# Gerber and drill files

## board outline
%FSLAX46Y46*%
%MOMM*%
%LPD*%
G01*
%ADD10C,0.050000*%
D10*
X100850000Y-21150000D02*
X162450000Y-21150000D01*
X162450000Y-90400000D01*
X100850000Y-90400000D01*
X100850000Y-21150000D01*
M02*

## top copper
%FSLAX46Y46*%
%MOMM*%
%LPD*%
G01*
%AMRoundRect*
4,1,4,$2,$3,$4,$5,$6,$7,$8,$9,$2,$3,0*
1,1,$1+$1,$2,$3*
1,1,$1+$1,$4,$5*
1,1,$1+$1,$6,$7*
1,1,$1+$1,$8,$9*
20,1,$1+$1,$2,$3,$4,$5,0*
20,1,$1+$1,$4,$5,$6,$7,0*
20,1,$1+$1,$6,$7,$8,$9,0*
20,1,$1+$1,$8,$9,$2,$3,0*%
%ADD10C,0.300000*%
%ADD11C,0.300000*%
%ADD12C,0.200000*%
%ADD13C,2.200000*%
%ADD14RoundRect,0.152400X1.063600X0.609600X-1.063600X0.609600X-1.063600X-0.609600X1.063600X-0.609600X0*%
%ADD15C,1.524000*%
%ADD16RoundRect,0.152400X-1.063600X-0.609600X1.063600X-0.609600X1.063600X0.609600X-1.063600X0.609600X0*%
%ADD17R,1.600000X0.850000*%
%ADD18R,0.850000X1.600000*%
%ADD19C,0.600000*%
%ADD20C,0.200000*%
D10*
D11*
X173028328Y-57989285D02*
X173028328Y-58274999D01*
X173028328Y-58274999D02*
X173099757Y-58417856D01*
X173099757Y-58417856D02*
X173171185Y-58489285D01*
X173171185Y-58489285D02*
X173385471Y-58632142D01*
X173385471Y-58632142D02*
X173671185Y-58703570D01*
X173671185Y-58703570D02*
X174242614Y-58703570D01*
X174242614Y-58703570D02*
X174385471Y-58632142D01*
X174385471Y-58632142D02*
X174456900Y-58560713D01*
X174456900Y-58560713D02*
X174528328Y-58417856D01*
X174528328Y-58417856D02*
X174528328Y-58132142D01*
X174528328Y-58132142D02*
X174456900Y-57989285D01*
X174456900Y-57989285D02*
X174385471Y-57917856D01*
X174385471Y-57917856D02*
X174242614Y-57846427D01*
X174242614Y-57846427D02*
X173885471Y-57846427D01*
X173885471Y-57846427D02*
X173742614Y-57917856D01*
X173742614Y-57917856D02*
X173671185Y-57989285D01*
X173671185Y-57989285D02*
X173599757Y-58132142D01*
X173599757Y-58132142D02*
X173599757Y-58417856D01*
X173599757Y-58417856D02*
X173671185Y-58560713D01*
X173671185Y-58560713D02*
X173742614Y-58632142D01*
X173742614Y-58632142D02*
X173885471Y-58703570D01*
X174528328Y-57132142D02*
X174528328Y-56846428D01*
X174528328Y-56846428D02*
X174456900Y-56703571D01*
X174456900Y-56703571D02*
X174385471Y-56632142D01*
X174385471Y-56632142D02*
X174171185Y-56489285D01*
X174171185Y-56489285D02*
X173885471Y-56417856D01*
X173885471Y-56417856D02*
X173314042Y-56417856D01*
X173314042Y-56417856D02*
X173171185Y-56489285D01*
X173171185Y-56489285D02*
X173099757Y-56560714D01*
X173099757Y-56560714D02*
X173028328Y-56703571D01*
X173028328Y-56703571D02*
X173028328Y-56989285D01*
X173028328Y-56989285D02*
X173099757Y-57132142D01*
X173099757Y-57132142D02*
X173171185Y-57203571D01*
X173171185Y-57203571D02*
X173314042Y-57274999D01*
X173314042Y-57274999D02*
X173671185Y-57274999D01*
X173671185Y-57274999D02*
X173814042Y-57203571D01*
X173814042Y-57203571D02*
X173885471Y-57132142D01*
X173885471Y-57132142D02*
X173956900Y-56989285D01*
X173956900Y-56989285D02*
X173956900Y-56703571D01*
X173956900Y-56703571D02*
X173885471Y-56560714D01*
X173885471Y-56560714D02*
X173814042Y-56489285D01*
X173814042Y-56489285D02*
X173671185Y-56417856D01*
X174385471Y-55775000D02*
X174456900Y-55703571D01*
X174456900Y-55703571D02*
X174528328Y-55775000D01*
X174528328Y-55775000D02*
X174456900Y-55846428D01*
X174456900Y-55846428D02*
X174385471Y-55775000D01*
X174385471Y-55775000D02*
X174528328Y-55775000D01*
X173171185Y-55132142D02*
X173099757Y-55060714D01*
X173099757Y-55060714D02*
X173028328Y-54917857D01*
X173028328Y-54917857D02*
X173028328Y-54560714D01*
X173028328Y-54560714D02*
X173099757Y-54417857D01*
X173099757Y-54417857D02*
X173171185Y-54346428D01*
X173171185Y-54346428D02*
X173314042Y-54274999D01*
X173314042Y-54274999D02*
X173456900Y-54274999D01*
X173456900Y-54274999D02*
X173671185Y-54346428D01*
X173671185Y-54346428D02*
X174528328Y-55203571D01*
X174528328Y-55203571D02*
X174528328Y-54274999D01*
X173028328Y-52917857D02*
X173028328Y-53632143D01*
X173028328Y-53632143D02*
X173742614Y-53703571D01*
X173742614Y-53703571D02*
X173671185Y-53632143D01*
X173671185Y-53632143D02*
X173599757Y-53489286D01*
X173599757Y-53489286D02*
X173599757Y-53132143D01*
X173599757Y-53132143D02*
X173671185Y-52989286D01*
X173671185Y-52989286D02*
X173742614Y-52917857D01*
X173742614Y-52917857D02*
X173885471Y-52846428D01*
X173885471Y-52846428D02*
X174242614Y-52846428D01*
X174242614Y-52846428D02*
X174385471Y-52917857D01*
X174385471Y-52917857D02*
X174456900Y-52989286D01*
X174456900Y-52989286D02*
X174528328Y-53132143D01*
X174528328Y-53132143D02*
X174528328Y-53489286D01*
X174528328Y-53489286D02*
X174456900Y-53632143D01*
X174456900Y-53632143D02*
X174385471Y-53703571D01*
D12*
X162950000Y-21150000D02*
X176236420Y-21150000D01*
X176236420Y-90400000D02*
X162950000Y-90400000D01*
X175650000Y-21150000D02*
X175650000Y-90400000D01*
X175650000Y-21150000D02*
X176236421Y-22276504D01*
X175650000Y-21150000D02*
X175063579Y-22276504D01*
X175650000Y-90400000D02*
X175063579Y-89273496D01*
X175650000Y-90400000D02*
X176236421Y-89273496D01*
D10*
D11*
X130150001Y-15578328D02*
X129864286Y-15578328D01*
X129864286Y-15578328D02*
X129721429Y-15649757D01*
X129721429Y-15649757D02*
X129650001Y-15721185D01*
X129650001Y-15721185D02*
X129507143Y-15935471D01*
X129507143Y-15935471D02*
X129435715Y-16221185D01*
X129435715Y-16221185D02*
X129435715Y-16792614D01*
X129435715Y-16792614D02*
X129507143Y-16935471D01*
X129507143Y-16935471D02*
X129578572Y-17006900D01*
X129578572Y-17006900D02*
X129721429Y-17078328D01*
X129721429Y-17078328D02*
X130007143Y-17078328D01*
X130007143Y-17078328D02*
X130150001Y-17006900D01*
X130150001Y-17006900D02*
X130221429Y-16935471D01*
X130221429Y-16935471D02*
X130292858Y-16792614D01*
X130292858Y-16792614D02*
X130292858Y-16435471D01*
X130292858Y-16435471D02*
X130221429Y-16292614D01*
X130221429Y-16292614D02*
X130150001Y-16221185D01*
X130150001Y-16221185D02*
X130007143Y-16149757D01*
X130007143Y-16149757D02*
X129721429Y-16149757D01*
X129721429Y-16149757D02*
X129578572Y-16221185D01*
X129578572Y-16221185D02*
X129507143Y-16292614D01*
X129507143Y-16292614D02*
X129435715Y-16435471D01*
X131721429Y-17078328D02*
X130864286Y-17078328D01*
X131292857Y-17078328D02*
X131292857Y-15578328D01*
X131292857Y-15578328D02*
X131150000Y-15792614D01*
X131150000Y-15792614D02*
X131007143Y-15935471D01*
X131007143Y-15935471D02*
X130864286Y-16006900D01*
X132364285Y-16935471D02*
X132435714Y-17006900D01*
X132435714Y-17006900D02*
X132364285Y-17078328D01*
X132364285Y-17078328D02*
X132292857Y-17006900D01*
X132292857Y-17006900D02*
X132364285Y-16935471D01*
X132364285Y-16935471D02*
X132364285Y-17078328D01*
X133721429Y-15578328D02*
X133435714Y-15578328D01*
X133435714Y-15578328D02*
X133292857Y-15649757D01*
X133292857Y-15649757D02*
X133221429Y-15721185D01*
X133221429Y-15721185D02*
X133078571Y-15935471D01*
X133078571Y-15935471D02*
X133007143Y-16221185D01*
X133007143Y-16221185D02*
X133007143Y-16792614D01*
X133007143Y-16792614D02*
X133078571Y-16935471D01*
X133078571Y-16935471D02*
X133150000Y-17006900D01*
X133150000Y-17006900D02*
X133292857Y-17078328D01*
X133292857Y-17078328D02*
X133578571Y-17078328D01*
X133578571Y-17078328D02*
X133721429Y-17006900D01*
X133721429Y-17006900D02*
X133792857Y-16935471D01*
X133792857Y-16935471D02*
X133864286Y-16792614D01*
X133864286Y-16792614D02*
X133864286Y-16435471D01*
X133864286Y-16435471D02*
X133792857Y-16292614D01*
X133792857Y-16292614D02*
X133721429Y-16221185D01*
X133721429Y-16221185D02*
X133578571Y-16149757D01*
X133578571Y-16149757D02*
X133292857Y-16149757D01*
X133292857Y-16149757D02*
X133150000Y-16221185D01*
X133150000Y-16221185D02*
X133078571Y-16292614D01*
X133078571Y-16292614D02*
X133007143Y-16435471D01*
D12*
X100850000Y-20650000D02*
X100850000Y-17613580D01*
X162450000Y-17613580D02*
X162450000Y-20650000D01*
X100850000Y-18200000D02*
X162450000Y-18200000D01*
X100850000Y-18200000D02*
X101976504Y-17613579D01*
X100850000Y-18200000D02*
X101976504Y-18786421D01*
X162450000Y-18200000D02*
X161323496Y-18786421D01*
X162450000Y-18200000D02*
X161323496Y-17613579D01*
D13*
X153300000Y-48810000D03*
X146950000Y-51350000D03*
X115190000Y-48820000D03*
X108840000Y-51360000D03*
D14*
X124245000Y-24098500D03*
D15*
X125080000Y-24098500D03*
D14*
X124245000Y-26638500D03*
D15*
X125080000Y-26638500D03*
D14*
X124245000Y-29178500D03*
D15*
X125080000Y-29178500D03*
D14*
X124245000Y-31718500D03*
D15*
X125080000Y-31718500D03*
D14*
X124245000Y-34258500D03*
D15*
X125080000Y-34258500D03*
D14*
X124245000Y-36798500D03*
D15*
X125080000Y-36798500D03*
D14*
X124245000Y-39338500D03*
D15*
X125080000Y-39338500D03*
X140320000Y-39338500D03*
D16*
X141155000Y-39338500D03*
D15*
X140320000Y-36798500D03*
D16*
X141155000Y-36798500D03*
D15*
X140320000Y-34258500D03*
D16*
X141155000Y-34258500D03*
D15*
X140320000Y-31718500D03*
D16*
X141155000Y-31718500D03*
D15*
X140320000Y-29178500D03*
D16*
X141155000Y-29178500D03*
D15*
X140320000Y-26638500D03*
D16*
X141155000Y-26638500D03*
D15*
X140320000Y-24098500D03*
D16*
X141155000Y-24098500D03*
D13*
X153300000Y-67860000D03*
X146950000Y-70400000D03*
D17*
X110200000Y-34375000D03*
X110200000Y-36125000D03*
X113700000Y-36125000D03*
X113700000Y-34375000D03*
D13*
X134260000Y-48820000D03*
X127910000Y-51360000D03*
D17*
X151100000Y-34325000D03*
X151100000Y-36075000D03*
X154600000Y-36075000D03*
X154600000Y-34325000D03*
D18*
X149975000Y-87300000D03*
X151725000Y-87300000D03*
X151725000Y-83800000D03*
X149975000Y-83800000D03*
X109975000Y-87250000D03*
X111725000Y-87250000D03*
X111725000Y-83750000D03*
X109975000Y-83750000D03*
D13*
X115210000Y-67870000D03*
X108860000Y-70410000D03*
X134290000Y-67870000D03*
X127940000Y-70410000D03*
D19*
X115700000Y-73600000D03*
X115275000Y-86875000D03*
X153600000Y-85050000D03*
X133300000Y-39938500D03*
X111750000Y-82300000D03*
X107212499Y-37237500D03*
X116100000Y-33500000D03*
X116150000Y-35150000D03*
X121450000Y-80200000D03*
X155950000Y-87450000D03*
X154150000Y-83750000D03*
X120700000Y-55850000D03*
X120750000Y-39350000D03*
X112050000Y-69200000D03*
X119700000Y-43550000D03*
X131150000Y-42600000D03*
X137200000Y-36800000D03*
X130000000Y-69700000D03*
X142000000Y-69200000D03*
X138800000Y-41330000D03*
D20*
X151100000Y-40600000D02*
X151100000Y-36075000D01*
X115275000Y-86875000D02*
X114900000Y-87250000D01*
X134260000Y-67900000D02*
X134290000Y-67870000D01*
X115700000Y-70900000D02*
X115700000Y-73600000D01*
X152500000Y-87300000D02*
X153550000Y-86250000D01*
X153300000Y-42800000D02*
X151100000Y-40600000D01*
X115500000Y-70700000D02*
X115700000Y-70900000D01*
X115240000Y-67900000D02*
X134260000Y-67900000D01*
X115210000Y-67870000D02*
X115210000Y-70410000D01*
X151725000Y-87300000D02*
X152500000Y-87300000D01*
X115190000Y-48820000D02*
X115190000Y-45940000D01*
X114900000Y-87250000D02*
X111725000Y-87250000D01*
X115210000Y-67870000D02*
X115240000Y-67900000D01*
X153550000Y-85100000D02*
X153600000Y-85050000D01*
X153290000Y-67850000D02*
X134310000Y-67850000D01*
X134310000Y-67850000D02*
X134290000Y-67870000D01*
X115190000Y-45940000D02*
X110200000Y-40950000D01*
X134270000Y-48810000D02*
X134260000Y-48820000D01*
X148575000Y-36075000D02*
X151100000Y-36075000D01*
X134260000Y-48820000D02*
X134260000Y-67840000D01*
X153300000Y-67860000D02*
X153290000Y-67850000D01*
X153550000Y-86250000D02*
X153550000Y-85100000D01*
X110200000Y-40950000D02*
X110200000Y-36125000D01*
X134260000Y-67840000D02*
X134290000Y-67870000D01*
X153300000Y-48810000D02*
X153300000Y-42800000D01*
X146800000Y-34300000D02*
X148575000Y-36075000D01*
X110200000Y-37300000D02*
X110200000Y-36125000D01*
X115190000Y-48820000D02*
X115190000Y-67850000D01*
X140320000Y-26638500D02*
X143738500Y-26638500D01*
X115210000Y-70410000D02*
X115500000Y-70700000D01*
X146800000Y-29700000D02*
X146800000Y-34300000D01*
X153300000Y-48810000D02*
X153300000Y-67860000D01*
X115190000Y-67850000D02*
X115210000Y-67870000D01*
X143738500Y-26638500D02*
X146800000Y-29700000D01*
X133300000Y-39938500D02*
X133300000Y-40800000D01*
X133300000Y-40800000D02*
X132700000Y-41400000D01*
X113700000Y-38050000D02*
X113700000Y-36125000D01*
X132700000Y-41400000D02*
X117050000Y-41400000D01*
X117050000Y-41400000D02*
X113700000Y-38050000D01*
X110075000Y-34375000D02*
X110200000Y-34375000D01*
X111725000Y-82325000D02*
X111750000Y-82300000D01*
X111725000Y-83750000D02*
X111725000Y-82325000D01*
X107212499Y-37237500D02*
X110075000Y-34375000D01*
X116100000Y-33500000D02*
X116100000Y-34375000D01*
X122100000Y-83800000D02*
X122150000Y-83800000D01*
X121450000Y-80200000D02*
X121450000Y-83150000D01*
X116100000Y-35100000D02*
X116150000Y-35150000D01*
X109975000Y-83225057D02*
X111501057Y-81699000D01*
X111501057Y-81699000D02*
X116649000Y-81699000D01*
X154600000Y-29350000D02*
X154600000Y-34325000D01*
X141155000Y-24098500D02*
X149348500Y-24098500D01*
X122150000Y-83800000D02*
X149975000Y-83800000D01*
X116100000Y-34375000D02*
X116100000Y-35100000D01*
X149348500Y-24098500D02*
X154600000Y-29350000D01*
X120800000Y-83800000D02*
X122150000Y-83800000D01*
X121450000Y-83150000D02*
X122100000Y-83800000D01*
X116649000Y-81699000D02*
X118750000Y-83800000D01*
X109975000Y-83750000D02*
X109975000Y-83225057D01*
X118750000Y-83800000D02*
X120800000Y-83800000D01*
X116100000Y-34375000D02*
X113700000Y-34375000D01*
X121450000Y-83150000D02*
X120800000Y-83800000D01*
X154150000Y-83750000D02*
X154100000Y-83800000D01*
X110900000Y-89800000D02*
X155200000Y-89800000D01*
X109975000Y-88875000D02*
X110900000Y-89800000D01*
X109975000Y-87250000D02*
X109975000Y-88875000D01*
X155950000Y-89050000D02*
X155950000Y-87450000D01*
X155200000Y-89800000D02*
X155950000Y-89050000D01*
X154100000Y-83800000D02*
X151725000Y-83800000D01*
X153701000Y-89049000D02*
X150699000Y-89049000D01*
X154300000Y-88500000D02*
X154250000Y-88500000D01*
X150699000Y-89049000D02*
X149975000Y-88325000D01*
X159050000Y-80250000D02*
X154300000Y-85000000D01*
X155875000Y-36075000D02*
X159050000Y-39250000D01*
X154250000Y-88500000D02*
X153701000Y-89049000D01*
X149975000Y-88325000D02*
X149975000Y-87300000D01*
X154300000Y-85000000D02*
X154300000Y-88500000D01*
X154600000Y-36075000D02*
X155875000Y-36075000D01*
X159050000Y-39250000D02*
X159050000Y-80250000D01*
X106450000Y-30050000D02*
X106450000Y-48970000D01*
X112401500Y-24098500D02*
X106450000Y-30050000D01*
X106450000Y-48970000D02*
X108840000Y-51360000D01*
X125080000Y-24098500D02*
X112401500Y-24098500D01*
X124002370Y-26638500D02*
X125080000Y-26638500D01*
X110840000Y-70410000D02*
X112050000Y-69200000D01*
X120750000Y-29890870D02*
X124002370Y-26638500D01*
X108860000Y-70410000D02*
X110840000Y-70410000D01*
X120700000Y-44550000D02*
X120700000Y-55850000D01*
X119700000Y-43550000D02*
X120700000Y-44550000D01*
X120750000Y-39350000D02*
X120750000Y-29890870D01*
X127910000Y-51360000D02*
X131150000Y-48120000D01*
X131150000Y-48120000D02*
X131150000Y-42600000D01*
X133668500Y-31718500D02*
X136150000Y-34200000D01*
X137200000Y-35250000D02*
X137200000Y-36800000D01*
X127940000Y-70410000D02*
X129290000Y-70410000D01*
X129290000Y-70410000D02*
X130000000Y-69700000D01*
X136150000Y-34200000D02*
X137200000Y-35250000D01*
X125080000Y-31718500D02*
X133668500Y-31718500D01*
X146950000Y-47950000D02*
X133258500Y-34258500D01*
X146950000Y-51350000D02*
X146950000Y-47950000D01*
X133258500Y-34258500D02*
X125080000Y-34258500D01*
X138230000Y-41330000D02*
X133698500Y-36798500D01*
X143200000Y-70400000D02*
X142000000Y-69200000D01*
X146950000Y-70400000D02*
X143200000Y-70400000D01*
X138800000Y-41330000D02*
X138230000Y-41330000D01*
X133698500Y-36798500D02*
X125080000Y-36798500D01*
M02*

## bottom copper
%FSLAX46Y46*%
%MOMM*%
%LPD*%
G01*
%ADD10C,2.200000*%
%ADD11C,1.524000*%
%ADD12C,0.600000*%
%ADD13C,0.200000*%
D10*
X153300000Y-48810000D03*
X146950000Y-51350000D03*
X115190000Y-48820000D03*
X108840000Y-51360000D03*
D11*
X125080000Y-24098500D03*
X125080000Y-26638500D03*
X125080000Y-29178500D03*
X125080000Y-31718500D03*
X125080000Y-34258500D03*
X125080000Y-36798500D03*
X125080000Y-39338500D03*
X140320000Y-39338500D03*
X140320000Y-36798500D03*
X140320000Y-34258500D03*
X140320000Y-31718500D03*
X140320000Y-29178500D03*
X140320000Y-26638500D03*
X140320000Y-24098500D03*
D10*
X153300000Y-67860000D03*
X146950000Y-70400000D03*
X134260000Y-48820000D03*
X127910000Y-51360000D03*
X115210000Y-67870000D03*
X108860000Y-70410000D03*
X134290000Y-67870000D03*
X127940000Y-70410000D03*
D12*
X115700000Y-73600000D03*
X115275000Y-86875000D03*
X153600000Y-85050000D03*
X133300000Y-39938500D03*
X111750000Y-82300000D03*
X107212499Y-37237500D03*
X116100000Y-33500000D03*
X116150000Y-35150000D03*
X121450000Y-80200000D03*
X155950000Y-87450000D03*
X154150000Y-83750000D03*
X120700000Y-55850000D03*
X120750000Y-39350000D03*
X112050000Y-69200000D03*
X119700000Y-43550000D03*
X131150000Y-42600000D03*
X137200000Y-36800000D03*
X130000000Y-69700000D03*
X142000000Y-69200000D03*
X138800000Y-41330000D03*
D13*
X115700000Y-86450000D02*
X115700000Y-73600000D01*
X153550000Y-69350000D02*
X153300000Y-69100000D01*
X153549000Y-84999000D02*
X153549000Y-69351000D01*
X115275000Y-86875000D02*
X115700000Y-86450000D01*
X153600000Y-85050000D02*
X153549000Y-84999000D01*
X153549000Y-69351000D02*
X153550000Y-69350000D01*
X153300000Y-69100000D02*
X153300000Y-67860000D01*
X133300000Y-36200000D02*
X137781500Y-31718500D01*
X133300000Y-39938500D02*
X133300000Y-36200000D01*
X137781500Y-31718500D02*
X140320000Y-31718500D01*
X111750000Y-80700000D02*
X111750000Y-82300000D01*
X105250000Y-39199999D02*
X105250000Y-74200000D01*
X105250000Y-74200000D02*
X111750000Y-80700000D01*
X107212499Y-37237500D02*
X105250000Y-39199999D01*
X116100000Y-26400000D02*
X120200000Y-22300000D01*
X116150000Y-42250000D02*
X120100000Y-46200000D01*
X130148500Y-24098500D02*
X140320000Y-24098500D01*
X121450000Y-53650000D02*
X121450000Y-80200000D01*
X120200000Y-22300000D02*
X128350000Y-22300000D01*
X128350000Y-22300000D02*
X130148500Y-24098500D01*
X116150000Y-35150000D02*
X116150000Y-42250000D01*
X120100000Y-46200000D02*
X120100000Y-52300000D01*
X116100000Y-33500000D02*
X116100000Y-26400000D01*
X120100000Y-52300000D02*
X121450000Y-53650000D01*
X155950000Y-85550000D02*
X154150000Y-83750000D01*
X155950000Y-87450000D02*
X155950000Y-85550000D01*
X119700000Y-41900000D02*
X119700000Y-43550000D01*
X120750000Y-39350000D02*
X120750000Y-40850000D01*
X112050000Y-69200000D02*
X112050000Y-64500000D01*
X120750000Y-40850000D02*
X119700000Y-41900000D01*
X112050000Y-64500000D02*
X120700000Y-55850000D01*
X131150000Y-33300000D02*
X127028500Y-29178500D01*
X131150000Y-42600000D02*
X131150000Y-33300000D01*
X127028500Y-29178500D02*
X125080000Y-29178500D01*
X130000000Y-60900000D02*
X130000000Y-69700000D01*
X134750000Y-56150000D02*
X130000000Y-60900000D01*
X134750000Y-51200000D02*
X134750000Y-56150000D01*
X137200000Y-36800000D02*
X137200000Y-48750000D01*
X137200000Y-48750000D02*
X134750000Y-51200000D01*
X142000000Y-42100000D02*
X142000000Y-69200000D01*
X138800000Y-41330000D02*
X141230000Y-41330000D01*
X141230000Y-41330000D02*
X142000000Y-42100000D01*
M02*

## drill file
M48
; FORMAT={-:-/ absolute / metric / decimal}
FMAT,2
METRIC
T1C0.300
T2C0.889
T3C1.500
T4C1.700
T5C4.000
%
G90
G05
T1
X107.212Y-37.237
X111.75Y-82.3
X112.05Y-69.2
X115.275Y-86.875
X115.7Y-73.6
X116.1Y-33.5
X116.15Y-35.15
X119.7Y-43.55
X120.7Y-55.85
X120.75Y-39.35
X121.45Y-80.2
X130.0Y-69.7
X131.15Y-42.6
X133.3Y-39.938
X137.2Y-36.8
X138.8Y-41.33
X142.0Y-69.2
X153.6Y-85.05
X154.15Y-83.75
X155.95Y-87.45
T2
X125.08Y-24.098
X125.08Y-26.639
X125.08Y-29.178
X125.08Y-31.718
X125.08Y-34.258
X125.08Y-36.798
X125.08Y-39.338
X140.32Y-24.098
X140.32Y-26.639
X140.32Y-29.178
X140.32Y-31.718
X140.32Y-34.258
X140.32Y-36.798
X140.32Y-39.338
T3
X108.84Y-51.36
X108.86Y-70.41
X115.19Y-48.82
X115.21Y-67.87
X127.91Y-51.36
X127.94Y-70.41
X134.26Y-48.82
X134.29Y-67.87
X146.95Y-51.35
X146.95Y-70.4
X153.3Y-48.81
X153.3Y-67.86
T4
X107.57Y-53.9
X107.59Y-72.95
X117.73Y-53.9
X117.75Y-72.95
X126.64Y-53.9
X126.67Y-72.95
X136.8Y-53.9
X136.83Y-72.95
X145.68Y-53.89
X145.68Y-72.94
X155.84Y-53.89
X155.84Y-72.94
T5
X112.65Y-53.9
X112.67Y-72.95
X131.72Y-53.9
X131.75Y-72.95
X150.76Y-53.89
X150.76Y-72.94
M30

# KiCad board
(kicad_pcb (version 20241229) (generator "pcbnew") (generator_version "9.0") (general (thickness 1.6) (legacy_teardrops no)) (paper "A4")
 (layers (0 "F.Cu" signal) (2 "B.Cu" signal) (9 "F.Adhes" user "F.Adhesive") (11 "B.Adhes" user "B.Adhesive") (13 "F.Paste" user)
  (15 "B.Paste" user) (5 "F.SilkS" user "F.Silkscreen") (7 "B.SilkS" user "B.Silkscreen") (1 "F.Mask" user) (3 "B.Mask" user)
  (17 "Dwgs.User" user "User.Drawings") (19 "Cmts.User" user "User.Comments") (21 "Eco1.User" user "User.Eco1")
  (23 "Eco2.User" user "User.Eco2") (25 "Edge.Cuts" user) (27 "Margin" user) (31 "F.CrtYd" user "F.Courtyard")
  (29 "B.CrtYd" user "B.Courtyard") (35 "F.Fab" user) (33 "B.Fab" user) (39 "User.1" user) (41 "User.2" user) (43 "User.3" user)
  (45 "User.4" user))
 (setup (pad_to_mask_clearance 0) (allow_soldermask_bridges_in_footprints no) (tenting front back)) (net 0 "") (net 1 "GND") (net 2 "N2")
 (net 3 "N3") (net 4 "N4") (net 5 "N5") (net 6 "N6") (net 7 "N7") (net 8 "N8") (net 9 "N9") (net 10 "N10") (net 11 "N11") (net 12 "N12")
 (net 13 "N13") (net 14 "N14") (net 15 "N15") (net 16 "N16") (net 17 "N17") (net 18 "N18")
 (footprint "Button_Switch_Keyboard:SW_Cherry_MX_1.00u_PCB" (layer "F.Cu") (at 153.3 48.81)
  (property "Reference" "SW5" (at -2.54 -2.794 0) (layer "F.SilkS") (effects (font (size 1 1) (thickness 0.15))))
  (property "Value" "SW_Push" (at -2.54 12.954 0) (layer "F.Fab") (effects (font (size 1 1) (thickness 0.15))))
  (pad "" np_thru_hole circle (at -7.62 5.08) (size 1.7 1.7) (drill 1.7) (layers "*.Cu" "*.Mask"))
  (pad "" np_thru_hole circle (at -2.54 5.08) (size 4 4) (drill 4) (layers "*.Cu" "*.Mask"))
  (pad "" np_thru_hole circle (at 2.54 5.08) (size 1.7 1.7) (drill 1.7) (layers "*.Cu" "*.Mask"))
  (pad "1" thru_hole circle (at 0 0) (size 2.2 2.2) (drill 1.5) (layers "*.Cu" "*.Mask") (remove_unused_layers no) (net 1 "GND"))
  (pad "2" thru_hole circle (at -6.35 2.54) (size 2.2 2.2) (drill 1.5) (layers "*.Cu" "*.Mask") (remove_unused_layers no) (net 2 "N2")))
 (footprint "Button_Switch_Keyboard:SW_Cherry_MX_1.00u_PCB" (layer "F.Cu") (at 115.19 48.82)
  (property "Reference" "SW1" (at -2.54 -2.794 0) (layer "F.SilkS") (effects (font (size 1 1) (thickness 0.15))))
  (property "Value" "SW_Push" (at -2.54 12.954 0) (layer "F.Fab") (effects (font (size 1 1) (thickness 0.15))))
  (pad "" np_thru_hole circle (at -7.62 5.08) (size 1.7 1.7) (drill 1.7) (layers "*.Cu" "*.Mask"))
  (pad "" np_thru_hole circle (at -2.54 5.08) (size 4 4) (drill 4) (layers "*.Cu" "*.Mask"))
  (pad "" np_thru_hole circle (at 2.54 5.08) (size 1.7 1.7) (drill 1.7) (layers "*.Cu" "*.Mask"))
  (pad "1" thru_hole circle (at 0 0) (size 2.2 2.2) (drill 1.5) (layers "*.Cu" "*.Mask") (remove_unused_layers no) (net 1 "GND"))
  (pad "2" thru_hole circle (at -6.35 2.54) (size 2.2 2.2) (drill 1.5) (layers "*.Cu" "*.Mask") (remove_unused_layers no) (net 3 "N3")))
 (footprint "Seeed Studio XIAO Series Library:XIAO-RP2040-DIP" (layer "F.Cu") (at 132.7 31.7185)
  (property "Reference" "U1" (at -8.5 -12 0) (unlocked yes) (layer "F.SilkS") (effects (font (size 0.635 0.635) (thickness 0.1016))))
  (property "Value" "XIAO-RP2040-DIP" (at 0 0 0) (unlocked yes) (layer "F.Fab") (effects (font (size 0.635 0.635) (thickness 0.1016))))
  (pad "1" smd roundrect (at -8.455 -7.62 180) (size 2.432 1.524) (layers "F.Cu" "F.Mask") (roundrect_rratio 0.1) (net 3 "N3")
   (thermal_bridge_angle 45))
  (pad "1" thru_hole circle (at -7.62 -7.62 180) (size 1.524 1.524) (drill 0.889) (layers "*.Cu" "*.Mask") (remove_unused_layers no)
   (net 3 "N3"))
  (pad "2" smd roundrect (at -8.455 -5.08 180) (size 2.432 1.524) (layers "F.Cu" "F.Mask") (roundrect_rratio 0.1) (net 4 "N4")
   (thermal_bridge_angle 45))
  (pad "2" thru_hole circle (at -7.62 -5.08 180) (size 1.524 1.524) (drill 0.889) (layers "*.Cu" "*.Mask") (remove_unused_layers no)
   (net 4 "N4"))
  (pad "3" smd roundrect (at -8.455 -2.54 180) (size 2.432 1.524) (layers "F.Cu" "F.Mask") (roundrect_rratio 0.1) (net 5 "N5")
   (thermal_bridge_angle 45))
  (pad "3" thru_hole circle (at -7.62 -2.54 180) (size 1.524 1.524) (drill 0.889) (layers "*.Cu" "*.Mask") (remove_unused_layers no)
   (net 5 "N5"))
  (pad "4" smd roundrect (at -8.455 0 180) (size 2.432 1.524) (layers "F.Cu" "F.Mask") (roundrect_rratio 0.1) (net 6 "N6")
   (thermal_bridge_angle 45))
  (pad "4" thru_hole circle (at -7.62 0 180) (size 1.524 1.524) (drill 0.889) (layers "*.Cu" "*.Mask") (remove_unused_layers no)
   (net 6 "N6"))
  (pad "5" smd roundrect (at -8.455 2.54 180) (size 2.432 1.524) (layers "F.Cu" "F.Mask") (roundrect_rratio 0.1) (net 2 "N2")
   (thermal_bridge_angle 45))
  (pad "5" thru_hole circle (at -7.62 2.54 180) (size 1.524 1.524) (drill 0.889) (layers "*.Cu" "*.Mask") (remove_unused_layers no)
   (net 2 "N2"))
  (pad "6" smd roundrect (at -8.455 5.08 180) (size 2.432 1.524) (layers "F.Cu" "F.Mask") (roundrect_rratio 0.1) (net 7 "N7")
   (thermal_bridge_angle 45))
  (pad "6" thru_hole circle (at -7.62 5.08 180) (size 1.524 1.524) (drill 0.889) (layers "*.Cu" "*.Mask") (remove_unused_layers no)
   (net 7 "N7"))
  (pad "7" smd roundrect (at -8.455 7.62 180) (size 2.432 1.524) (layers "F.Cu" "F.Mask") (roundrect_rratio 0.1) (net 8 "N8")
   (thermal_bridge_angle 45))
  (pad "7" thru_hole circle (at -7.62 7.62 180) (size 1.524 1.524) (drill 0.889) (layers "*.Cu" "*.Mask") (remove_unused_layers no)
   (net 8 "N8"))
  (pad "8" thru_hole circle (at 7.62 7.62) (size 1.524 1.524) (drill 0.889) (layers "*.Cu" "*.Mask") (remove_unused_layers no) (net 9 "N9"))
  (pad "8" smd roundrect (at 8.455 7.62) (size 2.432 1.524) (layers "F.Cu" "F.Mask") (roundrect_rratio 0.1) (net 9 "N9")
   (thermal_bridge_angle 45))
  (pad "9" thru_hole circle (at 7.62 5.08) (size 1.524 1.524) (drill 0.889) (layers "*.Cu" "*.Mask") (remove_unused_layers no)
   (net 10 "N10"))
  (pad "9" smd roundrect (at 8.455 5.08) (size 2.432 1.524) (layers "F.Cu" "F.Mask") (roundrect_rratio 0.1) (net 10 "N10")
   (thermal_bridge_angle 45))
  (pad "10" thru_hole circle (at 7.62 2.54) (size 1.524 1.524) (drill 0.889) (layers "*.Cu" "*.Mask") (remove_unused_layers no)
   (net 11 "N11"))
  (pad "10" smd roundrect (at 8.455 2.54) (size 2.432 1.524) (layers "F.Cu" "F.Mask") (roundrect_rratio 0.1) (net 11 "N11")
   (thermal_bridge_angle 45))
  (pad "11" thru_hole circle (at 7.62 0) (size 1.524 1.524) (drill 0.889) (layers "*.Cu" "*.Mask") (remove_unused_layers no) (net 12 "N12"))
  (pad "11" smd roundrect (at 8.455 0) (size 2.432 1.524) (layers "F.Cu" "F.Mask") (roundrect_rratio 0.1) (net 12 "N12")
   (thermal_bridge_angle 45))
  (pad "12" thru_hole circle (at 7.62 -2.54) (size 1.524 1.524) (drill 0.889) (layers "*.Cu" "*.Mask") (remove_unused_layers no)
   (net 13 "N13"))
  (pad "12" smd roundrect (at 8.455 -2.54) (size 2.432 1.524) (layers "F.Cu" "F.Mask") (roundrect_rratio 0.1) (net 13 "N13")
   (thermal_bridge_angle 45))
  (pad "13" thru_hole circle (at 7.62 -5.08) (size 1.524 1.524) (drill 0.889) (layers "*.Cu" "*.Mask") (remove_unused_layers no)
   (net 1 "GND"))
  (pad "13" smd roundrect (at 8.455 -5.08) (size 2.432 1.524) (layers "F.Cu" "F.Mask") (roundrect_rratio 0.1) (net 1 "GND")
   (thermal_bridge_angle 45))
  (pad "14" thru_hole circle (at 7.62 -7.62) (size 1.524 1.524) (drill 0.889) (layers "*.Cu" "*.Mask") (remove_unused_layers no)
   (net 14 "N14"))
  (pad "14" smd roundrect (at 8.455 -7.62) (size 2.432 1.524) (layers "F.Cu" "F.Mask") (roundrect_rratio 0.1) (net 14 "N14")
   (thermal_bridge_angle 45)))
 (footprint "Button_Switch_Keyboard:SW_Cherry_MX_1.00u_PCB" (layer "F.Cu") (at 153.3 67.86)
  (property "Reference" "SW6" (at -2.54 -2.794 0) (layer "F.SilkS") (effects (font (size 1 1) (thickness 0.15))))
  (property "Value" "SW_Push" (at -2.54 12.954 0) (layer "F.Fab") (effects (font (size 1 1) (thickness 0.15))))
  (pad "" np_thru_hole circle (at -7.62 5.08) (size 1.7 1.7) (drill 1.7) (layers "*.Cu" "*.Mask"))
  (pad "" np_thru_hole circle (at -2.54 5.08) (size 4 4) (drill 4) (layers "*.Cu" "*.Mask"))
  (pad "" np_thru_hole circle (at 2.54 5.08) (size 1.7 1.7) (drill 1.7) (layers "*.Cu" "*.Mask"))
  (pad "1" thru_hole circle (at 0 0) (size 2.2 2.2) (drill 1.5) (layers "*.Cu" "*.Mask") (remove_unused_layers no) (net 1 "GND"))
  (pad "2" thru_hole circle (at -6.35 2.54) (size 2.2 2.2) (drill 1.5) (layers "*.Cu" "*.Mask") (remove_unused_layers no) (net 7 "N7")))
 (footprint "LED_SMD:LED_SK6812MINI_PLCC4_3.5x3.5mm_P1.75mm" (layer "F.Cu") (at 111.95 35.25)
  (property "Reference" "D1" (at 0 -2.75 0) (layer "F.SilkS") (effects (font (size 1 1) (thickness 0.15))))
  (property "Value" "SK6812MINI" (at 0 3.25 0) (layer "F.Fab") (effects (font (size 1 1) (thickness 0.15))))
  (pad "1" smd rect (at -1.75 -0.875) (size 1.6 0.85) (layers "F.Cu" "F.Mask" "F.Paste") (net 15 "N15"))
  (pad "2" smd rect (at -1.75 0.875) (size 1.6 0.85) (layers "F.Cu" "F.Mask" "F.Paste") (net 1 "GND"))
  (pad "3" smd rect (at 1.75 0.875) (size 1.6 0.85) (layers "F.Cu" "F.Mask" "F.Paste") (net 12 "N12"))
  (pad "4" smd rect (at 1.75 -0.875) (size 1.6 0.85) (layers "F.Cu" "F.Mask" "F.Paste") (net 14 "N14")))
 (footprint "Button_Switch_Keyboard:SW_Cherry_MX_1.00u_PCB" (layer "F.Cu") (at 134.26 48.82)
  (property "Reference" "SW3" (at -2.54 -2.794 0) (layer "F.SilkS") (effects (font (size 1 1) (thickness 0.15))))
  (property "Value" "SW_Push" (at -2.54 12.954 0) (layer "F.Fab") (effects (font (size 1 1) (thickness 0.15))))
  (pad "" np_thru_hole circle (at -7.62 5.08) (size 1.7 1.7) (drill 1.7) (layers "*.Cu" "*.Mask"))
  (pad "" np_thru_hole circle (at -2.54 5.08) (size 4 4) (drill 4) (layers "*.Cu" "*.Mask"))
  (pad "" np_thru_hole circle (at 2.54 5.08) (size 1.7 1.7) (drill 1.7) (layers "*.Cu" "*.Mask"))
  (pad "1" thru_hole circle (at 0 0) (size 2.2 2.2) (drill 1.5) (layers "*.Cu" "*.Mask") (remove_unused_layers no) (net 1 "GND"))
  (pad "2" thru_hole circle (at -6.35 2.54) (size 2.2 2.2) (drill 1.5) (layers "*.Cu" "*.Mask") (remove_unused_layers no) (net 5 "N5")))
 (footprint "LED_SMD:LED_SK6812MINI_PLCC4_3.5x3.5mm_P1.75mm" (layer "F.Cu") (at 152.85 35.2)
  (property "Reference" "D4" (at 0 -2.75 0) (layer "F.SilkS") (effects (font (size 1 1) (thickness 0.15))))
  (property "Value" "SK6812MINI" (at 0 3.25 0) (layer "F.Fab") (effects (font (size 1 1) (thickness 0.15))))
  (pad "1" smd rect (at -1.75 -0.875) (size 1.6 0.85) (layers "F.Cu" "F.Mask" "F.Paste") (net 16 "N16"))
  (pad "2" smd rect (at -1.75 0.875) (size 1.6 0.85) (layers "F.Cu" "F.Mask" "F.Paste") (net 1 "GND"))
  (pad "3" smd rect (at 1.75 0.875) (size 1.6 0.85) (layers "F.Cu" "F.Mask" "F.Paste") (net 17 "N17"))
  (pad "4" smd rect (at 1.75 -0.875) (size 1.6 0.85) (layers "F.Cu" "F.Mask" "F.Paste") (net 14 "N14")))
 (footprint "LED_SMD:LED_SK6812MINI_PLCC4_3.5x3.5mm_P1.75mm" (layer "F.Cu") (at 150.85 85.55 90)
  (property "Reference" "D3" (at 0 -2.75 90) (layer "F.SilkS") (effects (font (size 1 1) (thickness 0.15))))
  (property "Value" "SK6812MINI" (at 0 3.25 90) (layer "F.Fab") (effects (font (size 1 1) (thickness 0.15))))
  (pad "1" smd rect (at -1.75 -0.875 90) (size 1.6 0.85) (layers "F.Cu" "F.Mask" "F.Paste") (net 17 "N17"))
  (pad "2" smd rect (at -1.75 0.875 90) (size 1.6 0.85) (layers "F.Cu" "F.Mask" "F.Paste") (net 1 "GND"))
  (pad "3" smd rect (at 1.75 0.875 90) (size 1.6 0.85) (layers "F.Cu" "F.Mask" "F.Paste") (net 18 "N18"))
  (pad "4" smd rect (at 1.75 -0.875 90) (size 1.6 0.85) (layers "F.Cu" "F.Mask" "F.Paste") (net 14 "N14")))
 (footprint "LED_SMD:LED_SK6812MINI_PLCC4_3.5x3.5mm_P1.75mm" (layer "F.Cu") (at 110.85 85.5 90)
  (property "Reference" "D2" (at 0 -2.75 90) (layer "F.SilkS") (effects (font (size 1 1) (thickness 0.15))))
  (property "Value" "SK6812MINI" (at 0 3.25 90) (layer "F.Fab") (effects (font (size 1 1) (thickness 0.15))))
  (pad "1" smd rect (at -1.75 -0.875 90) (size 1.6 0.85) (layers "F.Cu" "F.Mask" "F.Paste") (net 18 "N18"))
  (pad "2" smd rect (at -1.75 0.875 90) (size 1.6 0.85) (layers "F.Cu" "F.Mask" "F.Paste") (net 1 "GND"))
  (pad "3" smd rect (at 1.75 0.875 90) (size 1.6 0.85) (layers "F.Cu" "F.Mask" "F.Paste") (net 15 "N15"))
  (pad "4" smd rect (at 1.75 -0.875 90) (size 1.6 0.85) (layers "F.Cu" "F.Mask" "F.Paste") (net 14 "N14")))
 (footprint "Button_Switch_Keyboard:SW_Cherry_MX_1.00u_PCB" (layer "F.Cu") (at 115.21 67.87)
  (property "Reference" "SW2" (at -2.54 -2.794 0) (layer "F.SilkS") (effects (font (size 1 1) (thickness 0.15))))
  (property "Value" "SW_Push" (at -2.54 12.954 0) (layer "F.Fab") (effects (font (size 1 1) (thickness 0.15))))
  (pad "" np_thru_hole circle (at -7.62 5.08) (size 1.7 1.7) (drill 1.7) (layers "*.Cu" "*.Mask"))
  (pad "" np_thru_hole circle (at -2.54 5.08) (size 4 4) (drill 4) (layers "*.Cu" "*.Mask"))
  (pad "" np_thru_hole circle (at 2.54 5.08) (size 1.7 1.7) (drill 1.7) (layers "*.Cu" "*.Mask"))
  (pad "1" thru_hole circle (at 0 0) (size 2.2 2.2) (drill 1.5) (layers "*.Cu" "*.Mask") (remove_unused_layers no) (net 1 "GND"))
  (pad "2" thru_hole circle (at -6.35 2.54) (size 2.2 2.2) (drill 1.5) (layers "*.Cu" "*.Mask") (remove_unused_layers no) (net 4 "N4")))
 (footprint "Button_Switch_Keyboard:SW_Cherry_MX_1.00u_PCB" (layer "F.Cu") (at 134.29 67.87)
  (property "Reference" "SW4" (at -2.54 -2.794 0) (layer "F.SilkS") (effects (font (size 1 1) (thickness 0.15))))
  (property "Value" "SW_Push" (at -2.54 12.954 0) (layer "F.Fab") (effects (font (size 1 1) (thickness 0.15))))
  (pad "" np_thru_hole circle (at -7.62 5.08) (size 1.7 1.7) (drill 1.7) (layers "*.Cu" "*.Mask"))
  (pad "" np_thru_hole circle (at -2.54 5.08) (size 4 4) (drill 4) (layers "*.Cu" "*.Mask"))
  (pad "" np_thru_hole circle (at 2.54 5.08) (size 1.7 1.7) (drill 1.7) (layers "*.Cu" "*.Mask"))
  (pad "1" thru_hole circle (at 0 0) (size 2.2 2.2) (drill 1.5) (layers "*.Cu" "*.Mask") (remove_unused_layers no) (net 1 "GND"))
  (pad "2" thru_hole circle (at -6.35 2.54) (size 2.2 2.2) (drill 1.5) (layers "*.Cu" "*.Mask") (remove_unused_layers no) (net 6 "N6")))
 (gr_rect (start 100.85 21.15) (end 162.45 90.4) (stroke (width 0.05) (type default)) (fill no) (layer "Edge.Cuts"))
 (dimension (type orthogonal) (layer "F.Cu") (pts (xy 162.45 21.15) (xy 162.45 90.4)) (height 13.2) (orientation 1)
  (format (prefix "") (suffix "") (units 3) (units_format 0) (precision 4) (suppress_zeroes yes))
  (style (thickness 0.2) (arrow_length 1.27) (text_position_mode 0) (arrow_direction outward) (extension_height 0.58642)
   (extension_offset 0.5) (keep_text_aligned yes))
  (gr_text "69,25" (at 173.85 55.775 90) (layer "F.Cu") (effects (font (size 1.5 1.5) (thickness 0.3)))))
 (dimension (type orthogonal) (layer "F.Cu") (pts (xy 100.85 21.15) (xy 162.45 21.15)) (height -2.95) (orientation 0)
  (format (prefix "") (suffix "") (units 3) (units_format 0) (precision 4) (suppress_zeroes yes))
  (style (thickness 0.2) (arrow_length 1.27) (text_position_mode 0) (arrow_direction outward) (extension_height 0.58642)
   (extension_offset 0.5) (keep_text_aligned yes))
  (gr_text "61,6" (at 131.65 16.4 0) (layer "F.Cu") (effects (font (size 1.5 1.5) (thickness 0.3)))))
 (segment (start 151.1 40.6) (end 151.1 36.075) (width 0.2) (layer "F.Cu") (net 1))
 (segment (start 115.275 86.875) (end 114.9 87.25) (width 0.2) (layer "F.Cu") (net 1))
 (segment (start 134.26 67.9) (end 134.29 67.87) (width 0.2) (layer "F.Cu") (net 1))
 (segment (start 115.7 70.9) (end 115.7 73.6) (width 0.2) (layer "F.Cu") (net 1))
 (segment (start 152.5 87.3) (end 153.55 86.25) (width 0.2) (layer "F.Cu") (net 1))
 (segment (start 153.3 42.8) (end 151.1 40.6) (width 0.2) (layer "F.Cu") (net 1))
 (segment (start 115.5 70.7) (end 115.7 70.9) (width 0.2) (layer "F.Cu") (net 1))
 (segment (start 115.24 67.9) (end 134.26 67.9) (width 0.2) (layer "F.Cu") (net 1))
 (segment (start 115.21 67.87) (end 115.21 70.41) (width 0.2) (layer "F.Cu") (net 1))
 (segment (start 151.725 87.3) (end 152.5 87.3) (width 0.2) (layer "F.Cu") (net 1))
 (segment (start 115.19 48.82) (end 115.19 45.94) (width 0.2) (layer "F.Cu") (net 1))
 (segment (start 114.9 87.25) (end 111.725 87.25) (width 0.2) (layer "F.Cu") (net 1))
 (segment (start 115.21 67.87) (end 115.24 67.9) (width 0.2) (layer "F.Cu") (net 1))
 (segment (start 153.55 85.1) (end 153.6 85.05) (width 0.2) (layer "F.Cu") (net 1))
 (segment (start 153.29 67.85) (end 134.31 67.85) (width 0.2) (layer "F.Cu") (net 1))
 (segment (start 134.31 67.85) (end 134.29 67.87) (width 0.2) (layer "F.Cu") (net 1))
 (segment (start 115.19 45.94) (end 110.2 40.95) (width 0.2) (layer "F.Cu") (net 1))
 (segment (start 134.27 48.81) (end 134.26 48.82) (width 0.2) (layer "F.Cu") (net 1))
 (segment (start 148.575 36.075) (end 151.1 36.075) (width 0.2) (layer "F.Cu") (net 1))
 (segment (start 134.26 48.82) (end 134.26 67.84) (width 0.2) (layer "F.Cu") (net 1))
 (segment (start 153.3 67.86) (end 153.29 67.85) (width 0.2) (layer "F.Cu") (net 1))
 (segment (start 153.55 86.25) (end 153.55 85.1) (width 0.2) (layer "F.Cu") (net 1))
 (segment (start 110.2 40.95) (end 110.2 36.125) (width 0.2) (layer "F.Cu") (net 1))
 (segment (start 134.26 67.84) (end 134.29 67.87) (width 0.2) (layer "F.Cu") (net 1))
 (segment (start 153.3 48.81) (end 153.3 42.8) (width 0.2) (layer "F.Cu") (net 1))
 (segment (start 146.8 34.3) (end 148.575 36.075) (width 0.2) (layer "F.Cu") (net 1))
 (segment (start 110.2 37.3) (end 110.2 36.125) (width 0.2) (layer "F.Cu") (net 1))
 (segment (start 115.19 48.82) (end 115.19 67.85) (width 0.2) (layer "F.Cu") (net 1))
 (segment (start 140.32 26.6385) (end 143.7385 26.6385) (width 0.2) (layer "F.Cu") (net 1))
 (segment (start 115.21 70.41) (end 115.5 70.7) (width 0.2) (layer "F.Cu") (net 1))
 (segment (start 146.8 29.7) (end 146.8 34.3) (width 0.2) (layer "F.Cu") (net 1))
 (segment (start 153.3 48.81) (end 153.3 67.86) (width 0.2) (layer "F.Cu") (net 1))
 (segment (start 115.19 67.85) (end 115.21 67.87) (width 0.2) (layer "F.Cu") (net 1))
 (segment (start 143.7385 26.6385) (end 146.8 29.7) (width 0.2) (layer "F.Cu") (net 1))
 (via (at 115.7 73.6) (size 0.6) (drill 0.3) (layers "F.Cu" "B.Cu") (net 1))
 (via (at 115.275 86.875) (size 0.6) (drill 0.3) (layers "F.Cu" "B.Cu") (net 1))
 (via (at 153.6 85.05) (size 0.6) (drill 0.3) (layers "F.Cu" "B.Cu") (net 1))
 (segment (start 115.7 86.45) (end 115.7 73.6) (width 0.2) (layer "B.Cu") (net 1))
 (segment (start 153.55 69.35) (end 153.3 69.1) (width 0.2) (layer "B.Cu") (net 1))
 (segment (start 153.549 84.999) (end 153.549 69.351) (width 0.2) (layer "B.Cu") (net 1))
 (segment (start 115.275 86.875) (end 115.7 86.45) (width 0.2) (layer "B.Cu") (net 1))
 (segment (start 153.6 85.05) (end 153.549 84.999) (width 0.2) (layer "B.Cu") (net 1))
 (segment (start 153.549 69.351) (end 153.55 69.35) (width 0.2) (layer "B.Cu") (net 1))
 (segment (start 153.3 69.1) (end 153.3 67.86) (width 0.2) (layer "B.Cu") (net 1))
 (segment (start 133.3 39.9385) (end 133.3 40.8) (width 0.2) (layer "F.Cu") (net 12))
 (segment (start 133.3 40.8) (end 132.7 41.4) (width 0.2) (layer "F.Cu") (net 12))
 (segment (start 113.7 38.05) (end 113.7 36.125) (width 0.2) (layer "F.Cu") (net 12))
 (segment (start 132.7 41.4) (end 117.05 41.4) (width 0.2) (layer "F.Cu") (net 12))
 (segment (start 117.05 41.4) (end 113.7 38.05) (width 0.2) (layer "F.Cu") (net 12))
 (via (at 133.3 39.9385) (size 0.6) (drill 0.3) (layers "F.Cu" "B.Cu") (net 12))
 (segment (start 133.3 36.2) (end 137.7815 31.7185) (width 0.2) (layer "B.Cu") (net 12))
 (segment (start 133.3 39.9385) (end 133.3 36.2) (width 0.2) (layer "B.Cu") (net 12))
 (segment (start 137.7815 31.7185) (end 140.32 31.7185) (width 0.2) (layer "B.Cu") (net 12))
 (segment (start 110.075 34.375) (end 110.2 34.375) (width 0.2) (layer "F.Cu") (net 15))
 (segment (start 111.725 82.325) (end 111.75 82.3) (width 0.2) (layer "F.Cu") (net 15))
 (segment (start 111.725 83.75) (end 111.725 82.325) (width 0.2) (layer "F.Cu") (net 15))
 (segment (start 107.212499 37.2375) (end 110.075 34.375) (width 0.2) (layer "F.Cu") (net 15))
 (via (at 111.75 82.3) (size 0.6) (drill 0.3) (layers "F.Cu" "B.Cu") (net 15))
 (via (at 107.212499 37.2375) (size 0.6) (drill 0.3) (layers "F.Cu" "B.Cu") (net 15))
 (segment (start 111.75 80.7) (end 111.75 82.3) (width 0.2) (layer "B.Cu") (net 15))
 (segment (start 105.25 39.199999) (end 105.25 74.2) (width 0.2) (layer "B.Cu") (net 15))
 (segment (start 105.25 74.2) (end 111.75 80.7) (width 0.2) (layer "B.Cu") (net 15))
 (segment (start 107.212499 37.2375) (end 105.25 39.199999) (width 0.2) (layer "B.Cu") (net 15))
 (segment (start 116.1 33.5) (end 116.1 34.375) (width 0.2) (layer "F.Cu") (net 14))
 (segment (start 122.1 83.8) (end 122.15 83.8) (width 0.2) (layer "F.Cu") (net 14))
 (segment (start 121.45 80.2) (end 121.45 83.15) (width 0.2) (layer "F.Cu") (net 14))
 (segment (start 116.1 35.1) (end 116.15 35.15) (width 0.2) (layer "F.Cu") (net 14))
 (segment (start 109.975 83.225057) (end 111.501057 81.699) (width 0.2) (layer "F.Cu") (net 14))
 (segment (start 111.501057 81.699) (end 116.649 81.699) (width 0.2) (layer "F.Cu") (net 14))
 (segment (start 154.6 29.35) (end 154.6 34.325) (width 0.2) (layer "F.Cu") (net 14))
 (segment (start 141.155 24.0985) (end 149.3485 24.0985) (width 0.2) (layer "F.Cu") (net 14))
 (segment (start 122.15 83.8) (end 149.975 83.8) (width 0.2) (layer "F.Cu") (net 14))
 (segment (start 116.1 34.375) (end 116.1 35.1) (width 0.2) (layer "F.Cu") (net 14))
 (segment (start 149.3485 24.0985) (end 154.6 29.35) (width 0.2) (layer "F.Cu") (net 14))
 (segment (start 120.8 83.8) (end 122.15 83.8) (width 0.2) (layer "F.Cu") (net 14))
 (segment (start 121.45 83.15) (end 122.1 83.8) (width 0.2) (layer "F.Cu") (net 14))
 (segment (start 116.649 81.699) (end 118.75 83.8) (width 0.2) (layer "F.Cu") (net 14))
 (segment (start 109.975 83.75) (end 109.975 83.225057) (width 0.2) (layer "F.Cu") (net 14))
 (segment (start 118.75 83.8) (end 120.8 83.8) (width 0.2) (layer "F.Cu") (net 14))
 (segment (start 116.1 34.375) (end 113.7 34.375) (width 0.2) (layer "F.Cu") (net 14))
 (segment (start 121.45 83.15) (end 120.8 83.8) (width 0.2) (layer "F.Cu") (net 14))
 (via (at 116.1 33.5) (size 0.6) (drill 0.3) (layers "F.Cu" "B.Cu") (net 14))
 (via (at 116.15 35.15) (size 0.6) (drill 0.3) (layers "F.Cu" "B.Cu") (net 14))
 (via (at 121.45 80.2) (size 0.6) (drill 0.3) (layers "F.Cu" "B.Cu") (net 14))
 (segment (start 116.1 26.4) (end 120.2 22.3) (width 0.2) (layer "B.Cu") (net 14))
 (segment (start 116.15 42.25) (end 120.1 46.2) (width 0.2) (layer "B.Cu") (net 14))
 (segment (start 130.1485 24.0985) (end 140.32 24.0985) (width 0.2) (layer "B.Cu") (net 14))
 (segment (start 121.45 53.65) (end 121.45 80.2) (width 0.2) (layer "B.Cu") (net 14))
 (segment (start 120.2 22.3) (end 128.35 22.3) (width 0.2) (layer "B.Cu") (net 14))
 (segment (start 128.35 22.3) (end 130.1485 24.0985) (width 0.2) (layer "B.Cu") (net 14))
 (segment (start 116.15 35.15) (end 116.15 42.25) (width 0.2) (layer "B.Cu") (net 14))
 (segment (start 120.1 46.2) (end 120.1 52.3) (width 0.2) (layer "B.Cu") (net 14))
 (segment (start 116.1 33.5) (end 116.1 26.4) (width 0.2) (layer "B.Cu") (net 14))
 (segment (start 120.1 52.3) (end 121.45 53.65) (width 0.2) (layer "B.Cu") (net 14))
 (segment (start 154.15 83.75) (end 154.1 83.8) (width 0.2) (layer "F.Cu") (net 18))
 (segment (start 110.9 89.8) (end 155.2 89.8) (width 0.2) (layer "F.Cu") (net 18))
 (segment (start 109.975 88.875) (end 110.9 89.8) (width 0.2) (layer "F.Cu") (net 18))
 (segment (start 109.975 87.25) (end 109.975 88.875) (width 0.2) (layer "F.Cu") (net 18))
 (segment (start 155.95 89.05) (end 155.95 87.45) (width 0.2) (layer "F.Cu") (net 18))
 (segment (start 155.2 89.8) (end 155.95 89.05) (width 0.2) (layer "F.Cu") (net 18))
 (segment (start 154.1 83.8) (end 151.725 83.8) (width 0.2) (layer "F.Cu") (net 18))
 (via (at 155.95 87.45) (size 0.6) (drill 0.3) (layers "F.Cu" "B.Cu") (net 18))
 (via (at 154.15 83.75) (size 0.6) (drill 0.3) (layers "F.Cu" "B.Cu") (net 18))
 (segment (start 155.95 85.55) (end 154.15 83.75) (width 0.2) (layer "B.Cu") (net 18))
 (segment (start 155.95 87.45) (end 155.95 85.55) (width 0.2) (layer "B.Cu") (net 18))
 (segment (start 153.701 89.049) (end 150.699 89.049) (width 0.2) (layer "F.Cu") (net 17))
 (segment (start 154.3 88.5) (end 154.25 88.5) (width 0.2) (layer "F.Cu") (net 17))
 (segment (start 150.699 89.049) (end 149.975 88.325) (width 0.2) (layer "F.Cu") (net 17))
 (segment (start 159.05 80.25) (end 154.3 85) (width 0.2) (layer "F.Cu") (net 17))
 (segment (start 155.875 36.075) (end 159.05 39.25) (width 0.2) (layer "F.Cu") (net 17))
 (segment (start 154.25 88.5) (end 153.701 89.049) (width 0.2) (layer "F.Cu") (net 17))
 (segment (start 149.975 88.325) (end 149.975 87.3) (width 0.2) (layer "F.Cu") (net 17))
 (segment (start 154.3 85) (end 154.3 88.5) (width 0.2) (layer "F.Cu") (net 17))
 (segment (start 154.6 36.075) (end 155.875 36.075) (width 0.2) (layer "F.Cu") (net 17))
 (segment (start 159.05 39.25) (end 159.05 80.25) (width 0.2) (layer "F.Cu") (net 17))
 (segment (start 106.45 30.05) (end 106.45 48.97) (width 0.2) (layer "F.Cu") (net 3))
 (segment (start 112.4015 24.0985) (end 106.45 30.05) (width 0.2) (layer "F.Cu") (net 3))
 (segment (start 106.45 48.97) (end 108.84 51.36) (width 0.2) (layer "F.Cu") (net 3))
 (segment (start 125.08 24.0985) (end 112.4015 24.0985) (width 0.2) (layer "F.Cu") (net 3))
 (segment (start 124.00237 26.6385) (end 125.08 26.6385) (width 0.2) (layer "F.Cu") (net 4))
 (segment (start 110.84 70.41) (end 112.05 69.2) (width 0.2) (layer "F.Cu") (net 4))
 (segment (start 120.75 29.89087) (end 124.00237 26.6385) (width 0.2) (layer "F.Cu") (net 4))
 (segment (start 108.86 70.41) (end 110.84 70.41) (width 0.2) (layer "F.Cu") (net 4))
 (segment (start 120.7 44.55) (end 120.7 55.85) (width 0.2) (layer "F.Cu") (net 4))
 (segment (start 119.7 43.55) (end 120.7 44.55) (width 0.2) (layer "F.Cu") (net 4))
 (segment (start 120.75 39.35) (end 120.75 29.89087) (width 0.2) (layer "F.Cu") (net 4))
 (via (at 120.7 55.85) (size 0.6) (drill 0.3) (layers "F.Cu" "B.Cu") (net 4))
 (via (at 120.75 39.35) (size 0.6) (drill 0.3) (layers "F.Cu" "B.Cu") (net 4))
 (via (at 112.05 69.2) (size 0.6) (drill 0.3) (layers "F.Cu" "B.Cu") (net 4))
 (via (at 119.7 43.55) (size 0.6) (drill 0.3) (layers "F.Cu" "B.Cu") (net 4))
 (segment (start 119.7 41.9) (end 119.7 43.55) (width 0.2) (layer "B.Cu") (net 4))
 (segment (start 120.75 39.35) (end 120.75 40.85) (width 0.2) (layer "B.Cu") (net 4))
 (segment (start 112.05 69.2) (end 112.05 64.5) (width 0.2) (layer "B.Cu") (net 4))
 (segment (start 120.75 40.85) (end 119.7 41.9) (width 0.2) (layer "B.Cu") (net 4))
 (segment (start 112.05 64.5) (end 120.7 55.85) (width 0.2) (layer "B.Cu") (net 4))
 (segment (start 127.91 51.36) (end 131.15 48.12) (width 0.2) (layer "F.Cu") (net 5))
 (segment (start 131.15 48.12) (end 131.15 42.6) (width 0.2) (layer "F.Cu") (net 5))
 (via (at 131.15 42.6) (size 0.6) (drill 0.3) (layers "F.Cu" "B.Cu") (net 5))
 (segment (start 131.15 33.3) (end 127.0285 29.1785) (width 0.2) (layer "B.Cu") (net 5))
 (segment (start 131.15 42.6) (end 131.15 33.3) (width 0.2) (layer "B.Cu") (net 5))
 (segment (start 127.0285 29.1785) (end 125.08 29.1785) (width 0.2) (layer "B.Cu") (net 5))
 (segment (start 133.6685 31.7185) (end 136.15 34.2) (width 0.2) (layer "F.Cu") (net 6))
 (segment (start 137.2 35.25) (end 137.2 36.8) (width 0.2) (layer "F.Cu") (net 6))
 (segment (start 127.94 70.41) (end 129.29 70.41) (width 0.2) (layer "F.Cu") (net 6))
 (segment (start 129.29 70.41) (end 130 69.7) (width 0.2) (layer "F.Cu") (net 6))
 (segment (start 136.15 34.2) (end 137.2 35.25) (width 0.2) (layer "F.Cu") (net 6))
 (segment (start 125.08 31.7185) (end 133.6685 31.7185) (width 0.2) (layer "F.Cu") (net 6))
 (via (at 137.2 36.8) (size 0.6) (drill 0.3) (layers "F.Cu" "B.Cu") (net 6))
 (via (at 130 69.7) (size 0.6) (drill 0.3) (layers "F.Cu" "B.Cu") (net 6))
 (segment (start 130 60.9) (end 130 69.7) (width 0.2) (layer "B.Cu") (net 6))
 (segment (start 134.75 56.15) (end 130 60.9) (width 0.2) (layer "B.Cu") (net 6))
 (segment (start 134.75 51.2) (end 134.75 56.15) (width 0.2) (layer "B.Cu") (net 6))
 (segment (start 137.2 36.8) (end 137.2 48.75) (width 0.2) (layer "B.Cu") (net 6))
 (segment (start 137.2 48.75) (end 134.75 51.2) (width 0.2) (layer "B.Cu") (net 6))
 (segment (start 146.95 47.95) (end 133.2585 34.2585) (width 0.2) (layer "F.Cu") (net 2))
 (segment (start 146.95 51.35) (end 146.95 47.95) (width 0.2) (layer "F.Cu") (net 2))
 (segment (start 133.2585 34.2585) (end 125.08 34.2585) (width 0.2) (layer "F.Cu") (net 2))
 (segment (start 138.23 41.33) (end 133.6985 36.7985) (width 0.2) (layer "F.Cu") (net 7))
 (segment (start 143.2 70.4) (end 142 69.2) (width 0.2) (layer "F.Cu") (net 7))
 (segment (start 146.95 70.4) (end 143.2 70.4) (width 0.2) (layer "F.Cu") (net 7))
 (segment (start 138.8 41.33) (end 138.23 41.33) (width 0.2) (layer "F.Cu") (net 7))
 (segment (start 133.6985 36.7985) (end 125.08 36.7985) (width 0.2) (layer "F.Cu") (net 7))
 (via (at 142 69.2) (size 0.6) (drill 0.3) (layers "F.Cu" "B.Cu") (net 7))
 (via (at 138.8 41.33) (size 0.6) (drill 0.3) (layers "F.Cu" "B.Cu") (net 7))
 (segment (start 142 42.1) (end 142 69.2) (width 0.2) (layer "B.Cu") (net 7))
 (segment (start 138.8 41.33) (end 141.23 41.33) (width 0.2) (layer "B.Cu") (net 7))
 (segment (start 141.23 41.33) (end 142 42.1) (width 0.2) (layer "B.Cu") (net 7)))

